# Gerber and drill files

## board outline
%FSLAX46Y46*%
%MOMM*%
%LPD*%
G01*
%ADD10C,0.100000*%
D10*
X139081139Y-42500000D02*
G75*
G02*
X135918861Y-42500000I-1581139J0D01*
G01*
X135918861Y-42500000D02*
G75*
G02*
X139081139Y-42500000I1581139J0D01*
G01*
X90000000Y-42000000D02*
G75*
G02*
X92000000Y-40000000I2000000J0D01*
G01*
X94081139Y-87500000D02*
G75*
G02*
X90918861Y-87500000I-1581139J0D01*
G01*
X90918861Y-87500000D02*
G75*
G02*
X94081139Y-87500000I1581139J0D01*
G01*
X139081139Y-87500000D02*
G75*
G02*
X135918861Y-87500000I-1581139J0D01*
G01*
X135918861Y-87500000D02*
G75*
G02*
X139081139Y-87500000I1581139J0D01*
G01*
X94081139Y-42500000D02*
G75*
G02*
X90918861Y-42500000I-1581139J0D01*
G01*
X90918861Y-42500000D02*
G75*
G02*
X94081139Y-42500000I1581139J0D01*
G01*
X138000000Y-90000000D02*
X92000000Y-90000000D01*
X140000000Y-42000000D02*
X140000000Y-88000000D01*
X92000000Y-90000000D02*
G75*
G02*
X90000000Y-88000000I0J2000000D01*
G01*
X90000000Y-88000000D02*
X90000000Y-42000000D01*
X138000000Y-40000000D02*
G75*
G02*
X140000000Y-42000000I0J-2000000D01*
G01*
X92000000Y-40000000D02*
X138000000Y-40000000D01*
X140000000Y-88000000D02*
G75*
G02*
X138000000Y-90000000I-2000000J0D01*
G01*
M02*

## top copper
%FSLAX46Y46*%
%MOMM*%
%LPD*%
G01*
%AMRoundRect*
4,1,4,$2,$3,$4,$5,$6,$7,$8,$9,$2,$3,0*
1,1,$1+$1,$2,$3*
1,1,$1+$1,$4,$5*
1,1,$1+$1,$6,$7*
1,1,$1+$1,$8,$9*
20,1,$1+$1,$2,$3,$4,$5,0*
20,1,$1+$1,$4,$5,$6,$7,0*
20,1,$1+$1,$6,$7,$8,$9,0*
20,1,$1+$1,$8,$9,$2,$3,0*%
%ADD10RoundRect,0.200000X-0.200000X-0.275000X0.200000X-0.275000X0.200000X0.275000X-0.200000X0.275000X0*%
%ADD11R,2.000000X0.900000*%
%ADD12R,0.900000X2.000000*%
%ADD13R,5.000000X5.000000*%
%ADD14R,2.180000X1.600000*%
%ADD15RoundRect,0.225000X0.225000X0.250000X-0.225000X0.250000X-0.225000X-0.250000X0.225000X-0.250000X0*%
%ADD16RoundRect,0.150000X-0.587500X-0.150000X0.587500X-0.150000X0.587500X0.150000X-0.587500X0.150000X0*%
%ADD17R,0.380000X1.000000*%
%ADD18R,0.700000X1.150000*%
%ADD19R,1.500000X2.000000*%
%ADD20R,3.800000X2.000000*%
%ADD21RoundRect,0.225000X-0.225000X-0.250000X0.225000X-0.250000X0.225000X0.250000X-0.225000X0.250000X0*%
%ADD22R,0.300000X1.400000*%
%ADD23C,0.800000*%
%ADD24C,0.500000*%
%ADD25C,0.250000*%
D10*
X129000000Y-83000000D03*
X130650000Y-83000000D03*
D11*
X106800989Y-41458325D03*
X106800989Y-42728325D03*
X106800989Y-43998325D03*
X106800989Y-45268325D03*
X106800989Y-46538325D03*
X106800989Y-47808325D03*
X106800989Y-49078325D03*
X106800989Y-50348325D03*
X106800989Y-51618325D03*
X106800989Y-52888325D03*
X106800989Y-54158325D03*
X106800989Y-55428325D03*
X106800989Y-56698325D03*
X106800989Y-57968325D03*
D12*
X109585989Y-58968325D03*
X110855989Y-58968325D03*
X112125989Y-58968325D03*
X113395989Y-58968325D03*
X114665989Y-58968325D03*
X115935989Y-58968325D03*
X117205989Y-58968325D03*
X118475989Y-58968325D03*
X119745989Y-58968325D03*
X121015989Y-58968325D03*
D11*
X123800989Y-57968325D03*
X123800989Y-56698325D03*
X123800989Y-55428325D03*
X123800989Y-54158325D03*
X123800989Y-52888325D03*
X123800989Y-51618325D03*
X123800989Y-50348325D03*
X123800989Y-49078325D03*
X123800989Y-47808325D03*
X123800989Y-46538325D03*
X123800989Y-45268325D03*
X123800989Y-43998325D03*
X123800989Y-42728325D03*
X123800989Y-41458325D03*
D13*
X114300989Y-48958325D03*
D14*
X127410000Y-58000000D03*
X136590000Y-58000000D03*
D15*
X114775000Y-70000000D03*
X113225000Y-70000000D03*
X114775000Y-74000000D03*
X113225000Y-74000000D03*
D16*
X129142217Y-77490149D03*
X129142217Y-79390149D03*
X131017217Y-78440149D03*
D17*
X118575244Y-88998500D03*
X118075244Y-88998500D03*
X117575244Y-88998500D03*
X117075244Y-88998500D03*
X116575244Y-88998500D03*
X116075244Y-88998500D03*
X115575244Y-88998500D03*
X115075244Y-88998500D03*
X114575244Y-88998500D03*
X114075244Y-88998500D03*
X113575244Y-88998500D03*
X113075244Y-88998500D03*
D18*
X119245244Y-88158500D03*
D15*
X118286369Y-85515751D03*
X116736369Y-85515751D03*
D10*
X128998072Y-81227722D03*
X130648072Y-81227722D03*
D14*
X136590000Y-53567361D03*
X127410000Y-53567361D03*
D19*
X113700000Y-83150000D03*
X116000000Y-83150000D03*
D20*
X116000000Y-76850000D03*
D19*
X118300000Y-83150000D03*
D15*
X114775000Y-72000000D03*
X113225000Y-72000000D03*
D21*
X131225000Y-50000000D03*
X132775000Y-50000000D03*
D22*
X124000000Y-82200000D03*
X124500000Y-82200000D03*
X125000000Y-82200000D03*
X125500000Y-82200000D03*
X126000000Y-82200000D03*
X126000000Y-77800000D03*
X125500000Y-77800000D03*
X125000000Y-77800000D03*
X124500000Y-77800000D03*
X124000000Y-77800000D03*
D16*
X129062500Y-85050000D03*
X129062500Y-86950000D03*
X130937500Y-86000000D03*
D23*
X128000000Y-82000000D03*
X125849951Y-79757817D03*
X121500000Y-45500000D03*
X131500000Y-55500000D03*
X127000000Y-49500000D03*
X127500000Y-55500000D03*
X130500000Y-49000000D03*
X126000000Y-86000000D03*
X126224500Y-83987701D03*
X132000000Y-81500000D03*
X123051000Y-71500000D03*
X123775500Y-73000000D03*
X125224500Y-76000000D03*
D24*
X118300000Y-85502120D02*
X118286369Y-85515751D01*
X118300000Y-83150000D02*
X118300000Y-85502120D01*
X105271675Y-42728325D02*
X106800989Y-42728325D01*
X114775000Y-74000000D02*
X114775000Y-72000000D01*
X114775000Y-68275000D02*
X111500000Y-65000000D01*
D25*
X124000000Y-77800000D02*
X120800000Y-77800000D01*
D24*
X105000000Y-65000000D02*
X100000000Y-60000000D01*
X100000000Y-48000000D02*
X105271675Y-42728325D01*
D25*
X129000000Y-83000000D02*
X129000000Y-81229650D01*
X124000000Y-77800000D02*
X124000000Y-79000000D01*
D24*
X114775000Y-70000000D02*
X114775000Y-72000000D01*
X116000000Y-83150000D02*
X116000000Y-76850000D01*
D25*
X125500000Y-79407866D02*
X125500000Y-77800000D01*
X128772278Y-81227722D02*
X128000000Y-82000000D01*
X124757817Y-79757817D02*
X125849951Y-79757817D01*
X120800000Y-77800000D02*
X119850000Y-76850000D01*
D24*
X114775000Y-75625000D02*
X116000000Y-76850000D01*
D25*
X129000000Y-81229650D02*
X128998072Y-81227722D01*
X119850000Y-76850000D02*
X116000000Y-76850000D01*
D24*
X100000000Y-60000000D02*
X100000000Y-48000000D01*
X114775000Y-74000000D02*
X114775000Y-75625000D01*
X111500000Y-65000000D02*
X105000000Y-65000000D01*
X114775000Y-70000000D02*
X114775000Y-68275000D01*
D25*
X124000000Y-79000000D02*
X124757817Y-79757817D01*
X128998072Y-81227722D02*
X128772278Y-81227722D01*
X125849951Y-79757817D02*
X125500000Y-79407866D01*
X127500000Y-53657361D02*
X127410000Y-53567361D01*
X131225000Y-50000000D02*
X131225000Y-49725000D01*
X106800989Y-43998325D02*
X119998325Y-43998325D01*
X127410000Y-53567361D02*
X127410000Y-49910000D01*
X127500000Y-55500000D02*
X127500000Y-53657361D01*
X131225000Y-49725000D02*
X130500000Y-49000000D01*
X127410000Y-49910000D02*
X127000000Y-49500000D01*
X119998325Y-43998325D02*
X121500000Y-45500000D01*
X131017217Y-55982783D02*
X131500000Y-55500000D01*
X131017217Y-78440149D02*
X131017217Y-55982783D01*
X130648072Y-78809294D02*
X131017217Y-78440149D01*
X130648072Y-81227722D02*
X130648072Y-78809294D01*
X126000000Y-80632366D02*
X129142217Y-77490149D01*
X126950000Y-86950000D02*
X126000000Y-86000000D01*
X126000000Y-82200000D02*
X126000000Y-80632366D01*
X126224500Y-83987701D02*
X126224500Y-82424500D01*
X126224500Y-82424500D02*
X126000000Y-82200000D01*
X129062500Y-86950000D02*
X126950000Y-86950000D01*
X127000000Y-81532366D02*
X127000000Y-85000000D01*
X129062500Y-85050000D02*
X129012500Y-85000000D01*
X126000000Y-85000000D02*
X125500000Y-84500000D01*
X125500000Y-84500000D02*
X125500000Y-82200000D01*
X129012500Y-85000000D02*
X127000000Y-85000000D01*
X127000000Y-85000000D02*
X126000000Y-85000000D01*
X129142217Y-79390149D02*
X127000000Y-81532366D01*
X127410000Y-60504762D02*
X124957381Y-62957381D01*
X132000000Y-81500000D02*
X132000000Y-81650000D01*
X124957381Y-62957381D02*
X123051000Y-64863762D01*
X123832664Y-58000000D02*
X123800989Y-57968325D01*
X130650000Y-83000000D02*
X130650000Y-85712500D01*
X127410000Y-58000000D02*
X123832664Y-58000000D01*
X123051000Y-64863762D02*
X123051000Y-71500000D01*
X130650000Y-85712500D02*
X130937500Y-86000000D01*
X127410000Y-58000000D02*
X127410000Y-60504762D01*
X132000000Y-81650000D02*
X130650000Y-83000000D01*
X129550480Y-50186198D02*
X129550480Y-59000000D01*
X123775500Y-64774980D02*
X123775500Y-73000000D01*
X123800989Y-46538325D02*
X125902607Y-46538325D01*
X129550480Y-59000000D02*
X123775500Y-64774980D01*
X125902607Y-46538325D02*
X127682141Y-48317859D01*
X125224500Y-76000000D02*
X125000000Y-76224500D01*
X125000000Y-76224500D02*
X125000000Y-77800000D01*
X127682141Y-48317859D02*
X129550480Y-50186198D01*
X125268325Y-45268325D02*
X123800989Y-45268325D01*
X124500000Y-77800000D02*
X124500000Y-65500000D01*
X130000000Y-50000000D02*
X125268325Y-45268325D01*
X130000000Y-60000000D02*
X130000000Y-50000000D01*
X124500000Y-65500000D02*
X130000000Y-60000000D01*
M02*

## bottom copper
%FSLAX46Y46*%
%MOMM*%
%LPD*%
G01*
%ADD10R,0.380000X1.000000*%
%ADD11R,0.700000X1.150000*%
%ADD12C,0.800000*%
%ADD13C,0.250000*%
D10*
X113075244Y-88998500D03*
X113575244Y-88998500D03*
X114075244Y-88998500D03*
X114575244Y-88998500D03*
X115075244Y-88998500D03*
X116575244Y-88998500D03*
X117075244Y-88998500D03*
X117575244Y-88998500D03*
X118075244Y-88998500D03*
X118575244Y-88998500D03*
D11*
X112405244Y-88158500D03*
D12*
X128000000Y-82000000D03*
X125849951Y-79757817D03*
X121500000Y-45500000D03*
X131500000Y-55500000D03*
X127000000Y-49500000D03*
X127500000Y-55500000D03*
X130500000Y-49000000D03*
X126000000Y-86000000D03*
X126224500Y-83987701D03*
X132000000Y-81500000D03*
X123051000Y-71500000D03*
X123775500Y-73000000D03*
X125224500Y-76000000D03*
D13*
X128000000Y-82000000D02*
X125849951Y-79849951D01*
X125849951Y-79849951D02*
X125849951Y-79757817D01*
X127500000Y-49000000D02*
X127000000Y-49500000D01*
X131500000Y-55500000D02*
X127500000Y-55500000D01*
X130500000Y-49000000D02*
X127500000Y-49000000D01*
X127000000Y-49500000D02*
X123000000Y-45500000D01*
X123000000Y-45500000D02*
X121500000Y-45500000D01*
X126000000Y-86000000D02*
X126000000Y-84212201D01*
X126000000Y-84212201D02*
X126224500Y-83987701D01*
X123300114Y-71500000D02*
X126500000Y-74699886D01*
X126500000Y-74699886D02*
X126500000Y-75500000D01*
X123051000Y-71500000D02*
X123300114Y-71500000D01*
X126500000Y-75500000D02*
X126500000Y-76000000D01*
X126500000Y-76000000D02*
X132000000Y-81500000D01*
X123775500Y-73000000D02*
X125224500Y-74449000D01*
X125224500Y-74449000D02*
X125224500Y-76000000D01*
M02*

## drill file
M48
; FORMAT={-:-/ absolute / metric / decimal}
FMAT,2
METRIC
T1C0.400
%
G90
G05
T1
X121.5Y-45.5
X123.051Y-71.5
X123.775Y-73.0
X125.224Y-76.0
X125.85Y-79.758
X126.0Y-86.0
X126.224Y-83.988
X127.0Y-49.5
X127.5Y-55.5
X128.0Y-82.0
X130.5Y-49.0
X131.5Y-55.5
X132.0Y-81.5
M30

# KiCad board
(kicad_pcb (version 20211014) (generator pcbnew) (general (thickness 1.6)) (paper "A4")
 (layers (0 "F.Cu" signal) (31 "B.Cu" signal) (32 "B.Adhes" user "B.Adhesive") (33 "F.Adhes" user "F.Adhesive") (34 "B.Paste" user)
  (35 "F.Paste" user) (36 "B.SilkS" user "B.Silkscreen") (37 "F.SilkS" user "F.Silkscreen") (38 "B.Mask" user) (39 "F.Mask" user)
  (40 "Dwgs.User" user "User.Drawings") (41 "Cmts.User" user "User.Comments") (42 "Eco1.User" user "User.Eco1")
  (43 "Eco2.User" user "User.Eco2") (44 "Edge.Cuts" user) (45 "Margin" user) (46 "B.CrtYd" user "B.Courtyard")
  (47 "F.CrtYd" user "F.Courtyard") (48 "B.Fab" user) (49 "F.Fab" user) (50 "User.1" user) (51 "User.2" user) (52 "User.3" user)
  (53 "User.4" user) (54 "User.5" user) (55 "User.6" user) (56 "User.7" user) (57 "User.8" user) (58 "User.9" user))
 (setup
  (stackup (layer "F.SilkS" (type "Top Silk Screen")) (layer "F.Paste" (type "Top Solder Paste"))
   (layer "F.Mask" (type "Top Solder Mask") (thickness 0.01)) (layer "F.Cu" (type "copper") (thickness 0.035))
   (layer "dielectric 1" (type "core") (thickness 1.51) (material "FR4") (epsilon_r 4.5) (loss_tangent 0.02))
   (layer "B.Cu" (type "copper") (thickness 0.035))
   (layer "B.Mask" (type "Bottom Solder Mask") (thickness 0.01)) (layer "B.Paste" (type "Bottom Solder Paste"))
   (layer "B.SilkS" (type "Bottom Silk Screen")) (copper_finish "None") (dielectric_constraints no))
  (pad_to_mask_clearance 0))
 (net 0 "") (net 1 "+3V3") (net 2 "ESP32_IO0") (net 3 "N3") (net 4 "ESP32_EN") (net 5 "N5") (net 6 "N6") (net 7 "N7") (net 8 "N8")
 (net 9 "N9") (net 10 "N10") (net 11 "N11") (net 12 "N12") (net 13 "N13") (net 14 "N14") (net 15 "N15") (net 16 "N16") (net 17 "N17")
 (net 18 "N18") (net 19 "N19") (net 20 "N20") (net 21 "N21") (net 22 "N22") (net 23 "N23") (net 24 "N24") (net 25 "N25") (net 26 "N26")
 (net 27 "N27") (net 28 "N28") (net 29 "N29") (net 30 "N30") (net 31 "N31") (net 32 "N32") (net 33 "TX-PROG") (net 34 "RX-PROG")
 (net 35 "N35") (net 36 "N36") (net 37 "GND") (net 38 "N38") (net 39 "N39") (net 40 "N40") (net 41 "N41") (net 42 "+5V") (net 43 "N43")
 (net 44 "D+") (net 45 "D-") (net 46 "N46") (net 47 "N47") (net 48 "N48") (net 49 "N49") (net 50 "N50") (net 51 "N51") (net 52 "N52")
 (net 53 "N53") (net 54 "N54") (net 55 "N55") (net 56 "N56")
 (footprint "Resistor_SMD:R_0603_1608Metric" (layer "F.Cu") (at 129.825 83)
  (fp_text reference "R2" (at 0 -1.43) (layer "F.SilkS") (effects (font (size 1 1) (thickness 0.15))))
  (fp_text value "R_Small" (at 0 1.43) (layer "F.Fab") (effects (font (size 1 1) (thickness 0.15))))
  (pad "1" smd roundrect (at -0.825 0) (size 0.8 0.95) (layers "F.Cu" "F.Paste" "F.Mask") (roundrect_rratio 0.25) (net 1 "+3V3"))
  (pad "2" smd roundrect (at 0.825 0) (size 0.8 0.95) (layers "F.Cu" "F.Paste" "F.Mask") (roundrect_rratio 0.25) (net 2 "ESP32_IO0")))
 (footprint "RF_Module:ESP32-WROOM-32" (layer "F.Cu") (at 115.300989 49.713325)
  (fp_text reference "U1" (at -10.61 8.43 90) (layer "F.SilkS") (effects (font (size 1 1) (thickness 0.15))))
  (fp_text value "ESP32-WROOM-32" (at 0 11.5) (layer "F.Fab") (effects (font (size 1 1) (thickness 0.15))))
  (pad "1" smd rect (at -8.5 -8.255) (size 2 0.9) (layers "F.Cu" "F.Paste" "F.Mask") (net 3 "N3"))
  (pad "2" smd rect (at -8.5 -6.985) (size 2 0.9) (layers "F.Cu" "F.Paste" "F.Mask") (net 1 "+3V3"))
  (pad "3" smd rect (at -8.5 -5.715) (size 2 0.9) (layers "F.Cu" "F.Paste" "F.Mask") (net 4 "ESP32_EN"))
  (pad "4" smd rect (at -8.5 -4.445) (size 2 0.9) (layers "F.Cu" "F.Paste" "F.Mask") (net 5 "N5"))
  (pad "5" smd rect (at -8.5 -3.175) (size 2 0.9) (layers "F.Cu" "F.Paste" "F.Mask") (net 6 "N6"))
  (pad "6" smd rect (at -8.5 -1.905) (size 2 0.9) (layers "F.Cu" "F.Paste" "F.Mask") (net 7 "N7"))
  (pad "7" smd rect (at -8.5 -0.635) (size 2 0.9) (layers "F.Cu" "F.Paste" "F.Mask") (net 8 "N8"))
  (pad "8" smd rect (at -8.5 0.635) (size 2 0.9) (layers "F.Cu" "F.Paste" "F.Mask") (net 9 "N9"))
  (pad "9" smd rect (at -8.5 1.905) (size 2 0.9) (layers "F.Cu" "F.Paste" "F.Mask") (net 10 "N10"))
  (pad "10" smd rect (at -8.5 3.175) (size 2 0.9) (layers "F.Cu" "F.Paste" "F.Mask") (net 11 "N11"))
  (pad "11" smd rect (at -8.5 4.445) (size 2 0.9) (layers "F.Cu" "F.Paste" "F.Mask") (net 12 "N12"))
  (pad "12" smd rect (at -8.5 5.715) (size 2 0.9) (layers "F.Cu" "F.Paste" "F.Mask") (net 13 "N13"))
  (pad "13" smd rect (at -8.5 6.985) (size 2 0.9) (layers "F.Cu" "F.Paste" "F.Mask") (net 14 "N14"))
  (pad "14" smd rect (at -8.5 8.255) (size 2 0.9) (layers "F.Cu" "F.Paste" "F.Mask") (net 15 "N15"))
  (pad "15" smd rect (at -5.715 9.255 90) (size 2 0.9) (layers "F.Cu" "F.Paste" "F.Mask") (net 3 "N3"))
  (pad "16" smd rect (at -4.445 9.255 90) (size 2 0.9) (layers "F.Cu" "F.Paste" "F.Mask") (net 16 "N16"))
  (pad "17" smd rect (at -3.175 9.255 90) (size 2 0.9) (layers "F.Cu" "F.Paste" "F.Mask") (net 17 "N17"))
  (pad "18" smd rect (at -1.905 9.255 90) (size 2 0.9) (layers "F.Cu" "F.Paste" "F.Mask") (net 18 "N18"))
  (pad "19" smd rect (at -0.635 9.255 90) (size 2 0.9) (layers "F.Cu" "F.Paste" "F.Mask") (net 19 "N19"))
  (pad "20" smd rect (at 0.635 9.255 90) (size 2 0.9) (layers "F.Cu" "F.Paste" "F.Mask") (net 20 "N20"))
  (pad "21" smd rect (at 1.905 9.255 90) (size 2 0.9) (layers "F.Cu" "F.Paste" "F.Mask") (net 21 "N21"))
  (pad "22" smd rect (at 3.175 9.255 90) (size 2 0.9) (layers "F.Cu" "F.Paste" "F.Mask") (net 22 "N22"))
  (pad "23" smd rect (at 4.445 9.255 90) (size 2 0.9) (layers "F.Cu" "F.Paste" "F.Mask") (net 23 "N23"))
  (pad "24" smd rect (at 5.715 9.255 90) (size 2 0.9) (layers "F.Cu" "F.Paste" "F.Mask") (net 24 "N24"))
  (pad "25" smd rect (at 8.5 8.255) (size 2 0.9) (layers "F.Cu" "F.Paste" "F.Mask") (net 2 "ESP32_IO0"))
  (pad "26" smd rect (at 8.5 6.985) (size 2 0.9) (layers "F.Cu" "F.Paste" "F.Mask") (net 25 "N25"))
  (pad "27" smd rect (at 8.5 5.715) (size 2 0.9) (layers "F.Cu" "F.Paste" "F.Mask") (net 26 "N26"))
  (pad "28" smd rect (at 8.5 4.445) (size 2 0.9) (layers "F.Cu" "F.Paste" "F.Mask") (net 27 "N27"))
  (pad "29" smd rect (at 8.5 3.175) (size 2 0.9) (layers "F.Cu" "F.Paste" "F.Mask") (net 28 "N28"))
  (pad "30" smd rect (at 8.5 1.905) (size 2 0.9) (layers "F.Cu" "F.Paste" "F.Mask") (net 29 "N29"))
  (pad "31" smd rect (at 8.5 0.635) (size 2 0.9) (layers "F.Cu" "F.Paste" "F.Mask") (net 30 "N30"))
  (pad "32" smd rect (at 8.5 -0.635) (size 2 0.9) (layers "F.Cu" "F.Paste" "F.Mask") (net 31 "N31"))
  (pad "33" smd rect (at 8.5 -1.905) (size 2 0.9) (layers "F.Cu" "F.Paste" "F.Mask") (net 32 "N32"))
  (pad "34" smd rect (at 8.5 -3.175) (size 2 0.9) (layers "F.Cu" "F.Paste" "F.Mask") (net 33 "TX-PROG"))
  (pad "35" smd rect (at 8.5 -4.445) (size 2 0.9) (layers "F.Cu" "F.Paste" "F.Mask") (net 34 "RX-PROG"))
  (pad "36" smd rect (at 8.5 -5.715) (size 2 0.9) (layers "F.Cu" "F.Paste" "F.Mask") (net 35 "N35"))
  (pad "37" smd rect (at 8.5 -6.985) (size 2 0.9) (layers "F.Cu" "F.Paste" "F.Mask") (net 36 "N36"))
  (pad "38" smd rect (at 8.5 -8.255) (size 2 0.9) (layers "F.Cu" "F.Paste" "F.Mask") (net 3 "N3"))
  (pad "39" smd rect (at -1 -0.755) (size 5 5) (layers "F.Cu" "F.Paste" "F.Mask") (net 3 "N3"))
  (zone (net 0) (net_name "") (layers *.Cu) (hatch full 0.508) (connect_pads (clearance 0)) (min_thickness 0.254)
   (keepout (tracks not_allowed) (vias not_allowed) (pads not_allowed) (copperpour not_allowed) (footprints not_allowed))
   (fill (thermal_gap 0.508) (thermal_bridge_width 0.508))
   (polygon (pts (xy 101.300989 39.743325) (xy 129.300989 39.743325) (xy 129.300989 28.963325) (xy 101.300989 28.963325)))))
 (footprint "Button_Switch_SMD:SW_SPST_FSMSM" (layer "F.Cu") (at 132 58)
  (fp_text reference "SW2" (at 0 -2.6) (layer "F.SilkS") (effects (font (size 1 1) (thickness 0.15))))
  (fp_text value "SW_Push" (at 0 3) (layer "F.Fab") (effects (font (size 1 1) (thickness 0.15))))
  (pad "1" smd rect (at -4.59 0) (size 2.18 1.6) (layers "F.Cu" "F.Paste" "F.Mask") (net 2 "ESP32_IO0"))
  (pad "2" smd rect (at 4.59 0) (size 2.18 1.6) (layers "F.Cu" "F.Paste" "F.Mask") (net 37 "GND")))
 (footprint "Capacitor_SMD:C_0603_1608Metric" (layer "F.Cu") (at 114 70 180)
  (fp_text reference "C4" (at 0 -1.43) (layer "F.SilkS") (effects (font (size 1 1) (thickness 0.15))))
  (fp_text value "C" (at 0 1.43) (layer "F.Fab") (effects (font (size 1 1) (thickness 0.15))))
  (pad "1" smd roundrect (at -0.775 0 180) (size 0.9 0.95) (layers "F.Cu" "F.Paste" "F.Mask") (roundrect_rratio 0.25) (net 1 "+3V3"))
  (pad "2" smd roundrect (at 0.775 0 180) (size 0.9 0.95) (layers "F.Cu" "F.Paste" "F.Mask") (roundrect_rratio 0.25) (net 37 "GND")))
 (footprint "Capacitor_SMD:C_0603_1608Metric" (layer "F.Cu") (at 114 74 180)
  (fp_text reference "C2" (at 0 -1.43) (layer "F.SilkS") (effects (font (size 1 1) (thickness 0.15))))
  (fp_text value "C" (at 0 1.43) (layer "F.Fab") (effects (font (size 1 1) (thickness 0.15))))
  (pad "1" smd roundrect (at -0.775 0 180) (size 0.9 0.95) (layers "F.Cu" "F.Paste" "F.Mask") (roundrect_rratio 0.25) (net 1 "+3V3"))
  (pad "2" smd roundrect (at 0.775 0 180) (size 0.9 0.95) (layers "F.Cu" "F.Paste" "F.Mask") (roundrect_rratio 0.25) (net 37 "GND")))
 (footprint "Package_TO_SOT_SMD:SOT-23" (layer "F.Cu") (at 130.079717 78.440149)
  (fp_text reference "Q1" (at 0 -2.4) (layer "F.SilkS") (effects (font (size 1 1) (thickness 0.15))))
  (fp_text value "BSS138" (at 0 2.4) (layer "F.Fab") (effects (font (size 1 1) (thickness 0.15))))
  (pad "1" smd roundrect (at -0.9375 -0.95) (size 1.475 0.6) (layers "F.Cu" "F.Paste" "F.Mask") (roundrect_rratio 0.25) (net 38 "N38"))
  (pad "2" smd roundrect (at -0.9375 0.95) (size 1.475 0.6) (layers "F.Cu" "F.Paste" "F.Mask") (roundrect_rratio 0.25) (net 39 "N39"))
  (pad "3" smd roundrect (at 0.9375 0) (size 1.475 0.6) (layers "F.Cu" "F.Paste" "F.Mask") (roundrect_rratio 0.25) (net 4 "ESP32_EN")))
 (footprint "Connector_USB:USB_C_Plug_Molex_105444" (layer "F.Cu") (at 115.825244 89.0385 180)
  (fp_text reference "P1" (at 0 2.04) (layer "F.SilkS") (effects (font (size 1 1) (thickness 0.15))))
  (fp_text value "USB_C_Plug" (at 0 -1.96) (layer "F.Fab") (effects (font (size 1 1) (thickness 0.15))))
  (pad "A1" smd rect (at -2.75 0.04 180) (size 0.38 1) (layers "F.Cu" "F.Paste" "F.Mask") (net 37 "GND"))
  (pad "A2" smd rect (at -2.25 0.04 180) (size 0.38 1) (layers "F.Cu" "F.Paste" "F.Mask") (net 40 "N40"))
  (pad "A3" smd rect (at -1.75 0.04 180) (size 0.38 1) (layers "F.Cu" "F.Paste" "F.Mask") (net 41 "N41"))
  (pad "A4" smd rect (at -1.25 0.04 180) (size 0.38 1) (layers "F.Cu" "F.Paste" "F.Mask") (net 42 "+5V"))
  (pad "A5" smd rect (at -0.75 0.04 180) (size 0.38 1) (layers "F.Cu" "F.Paste" "F.Mask") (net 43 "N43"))
  (pad "A6" smd rect (at -0.25 0.04 180) (size 0.38 1) (layers "F.Cu" "F.Paste" "F.Mask") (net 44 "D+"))
  (pad "A7" smd rect (at 0.25 0.04 180) (size 0.38 1) (layers "F.Cu" "F.Paste" "F.Mask") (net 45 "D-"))
  (pad "A8" smd rect (at 0.75 0.04 180) (size 0.38 1) (layers "F.Cu" "F.Paste" "F.Mask") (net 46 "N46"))
  (pad "A9" smd rect (at 1.25 0.04 180) (size 0.38 1) (layers "F.Cu" "F.Paste" "F.Mask") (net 42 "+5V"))
  (pad "A10" smd rect (at 1.75 0.04 180) (size 0.38 1) (layers "F.Cu" "F.Paste" "F.Mask") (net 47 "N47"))
  (pad "A11" smd rect (at 2.25 0.04 180) (size 0.38 1) (layers "F.Cu" "F.Paste" "F.Mask") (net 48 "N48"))
  (pad "A12" smd rect (at 2.75 0.04 180) (size 0.38 1) (layers "F.Cu" "F.Paste" "F.Mask") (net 37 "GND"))
  (pad "B1" smd rect (at 2.75 0.04 180) (size 0.38 1) (layers "B.Cu" "B.Paste" "B.Mask") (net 37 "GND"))
  (pad "B2" smd rect (at 2.25 0.04 180) (size 0.38 1) (layers "B.Cu" "B.Paste" "B.Mask") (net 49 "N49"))
  (pad "B3" smd rect (at 1.75 0.04 180) (size 0.38 1) (layers "B.Cu" "B.Paste" "B.Mask") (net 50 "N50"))
  (pad "B4" smd rect (at 1.25 0.04 180) (size 0.38 1) (layers "B.Cu" "B.Paste" "B.Mask") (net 42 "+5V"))
  (pad "B5" smd rect (at 0.75 0.04 180) (size 0.38 1) (layers "B.Cu" "B.Paste" "B.Mask") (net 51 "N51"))
  (pad "B8" smd rect (at -0.75 0.04 180) (size 0.38 1) (layers "B.Cu" "B.Paste" "B.Mask") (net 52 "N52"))
  (pad "B9" smd rect (at -1.25 0.04 180) (size 0.38 1) (layers "B.Cu" "B.Paste" "B.Mask") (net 42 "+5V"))
  (pad "B10" smd rect (at -1.75 0.04 180) (size 0.38 1) (layers "B.Cu" "B.Paste" "B.Mask") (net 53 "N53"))
  (pad "B11" smd rect (at -2.25 0.04 180) (size 0.38 1) (layers "B.Cu" "B.Paste" "B.Mask") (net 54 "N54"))
  (pad "B12" smd rect (at -2.75 0.04 180) (size 0.38 1) (layers "B.Cu" "B.Paste" "B.Mask") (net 37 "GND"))
  (pad "S1" smd rect (at 3.42 0.88 180) (size 0.7 1.15) (layers "B.Cu" "B.Paste" "B.Mask") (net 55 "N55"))
  (pad "S1" smd rect (at -3.42 0.88 180) (size 0.7 1.15) (layers "F.Cu" "F.Paste" "F.Mask") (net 55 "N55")))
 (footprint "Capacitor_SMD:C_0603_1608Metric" (layer "F.Cu") (at 117.511369 85.515751 180)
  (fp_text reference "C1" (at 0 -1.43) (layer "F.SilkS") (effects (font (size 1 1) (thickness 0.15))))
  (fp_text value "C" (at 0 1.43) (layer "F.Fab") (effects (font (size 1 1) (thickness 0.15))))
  (pad "1" smd roundrect (at -0.775 0 180) (size 0.9 0.95) (layers "F.Cu" "F.Paste" "F.Mask") (roundrect_rratio 0.25) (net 42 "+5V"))
  (pad "2" smd roundrect (at 0.775 0 180) (size 0.9 0.95) (layers "F.Cu" "F.Paste" "F.Mask") (roundrect_rratio 0.25) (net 37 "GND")))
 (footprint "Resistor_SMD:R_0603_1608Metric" (layer "F.Cu") (at 129.823072 81.227722)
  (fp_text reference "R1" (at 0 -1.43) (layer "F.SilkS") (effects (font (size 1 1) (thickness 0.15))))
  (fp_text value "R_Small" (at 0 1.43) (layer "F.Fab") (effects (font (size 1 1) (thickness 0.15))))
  (pad "1" smd roundrect (at -0.825 0) (size 0.8 0.95) (layers "F.Cu" "F.Paste" "F.Mask") (roundrect_rratio 0.25) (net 1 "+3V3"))
  (pad "2" smd roundrect (at 0.825 0) (size 0.8 0.95) (layers "F.Cu" "F.Paste" "F.Mask") (roundrect_rratio 0.25) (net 4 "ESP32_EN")))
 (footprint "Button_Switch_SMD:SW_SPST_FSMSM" (layer "F.Cu") (at 132 53.567361 180)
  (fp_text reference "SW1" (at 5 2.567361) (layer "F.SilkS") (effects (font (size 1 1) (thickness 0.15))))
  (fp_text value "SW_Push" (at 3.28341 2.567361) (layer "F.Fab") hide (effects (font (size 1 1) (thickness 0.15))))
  (pad "1" smd rect (at -4.59 0 180) (size 2.18 1.6) (layers "F.Cu" "F.Paste" "F.Mask") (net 37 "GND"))
  (pad "2" smd rect (at 4.59 0 180) (size 2.18 1.6) (layers "F.Cu" "F.Paste" "F.Mask") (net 4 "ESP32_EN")))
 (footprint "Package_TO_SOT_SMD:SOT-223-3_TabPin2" (layer "F.Cu") (at 116 80 90)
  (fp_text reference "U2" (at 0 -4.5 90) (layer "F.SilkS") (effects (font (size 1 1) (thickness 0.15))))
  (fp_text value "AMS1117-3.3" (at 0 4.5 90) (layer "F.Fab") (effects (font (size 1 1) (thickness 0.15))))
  (pad "1" smd rect (at -3.15 -2.3 90) (size 2 1.5) (layers "F.Cu" "F.Paste" "F.Mask") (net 37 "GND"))
  (pad "2" smd rect (at -3.15 0 90) (size 2 1.5) (layers "F.Cu" "F.Paste" "F.Mask") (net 1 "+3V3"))
  (pad "2" smd rect (at 3.15 0 90) (size 2 3.8) (layers "F.Cu" "F.Paste" "F.Mask") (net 1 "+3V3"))
  (pad "3" smd rect (at -3.15 2.3 90) (size 2 1.5) (layers "F.Cu" "F.Paste" "F.Mask") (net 42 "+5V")))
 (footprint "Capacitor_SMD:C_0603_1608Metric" (layer "F.Cu") (at 114 72 180)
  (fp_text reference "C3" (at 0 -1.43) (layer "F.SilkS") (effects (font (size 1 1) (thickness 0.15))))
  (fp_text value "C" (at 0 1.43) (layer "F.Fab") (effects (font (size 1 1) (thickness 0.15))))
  (pad "1" smd roundrect (at -0.775 0 180) (size 0.9 0.95) (layers "F.Cu" "F.Paste" "F.Mask") (roundrect_rratio 0.25) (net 1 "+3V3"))
  (pad "2" smd roundrect (at 0.775 0 180) (size 0.9 0.95) (layers "F.Cu" "F.Paste" "F.Mask") (roundrect_rratio 0.25) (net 37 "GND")))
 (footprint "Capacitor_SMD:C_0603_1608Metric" (layer "F.Cu") (at 132 50)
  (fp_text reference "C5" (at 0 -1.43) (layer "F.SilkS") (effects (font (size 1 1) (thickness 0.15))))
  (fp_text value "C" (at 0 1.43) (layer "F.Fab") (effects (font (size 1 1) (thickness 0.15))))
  (pad "1" smd roundrect (at -0.775 0) (size 0.9 0.95) (layers "F.Cu" "F.Paste" "F.Mask") (roundrect_rratio 0.25) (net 4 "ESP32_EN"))
  (pad "2" smd roundrect (at 0.775 0) (size 0.9 0.95) (layers "F.Cu" "F.Paste" "F.Mask") (roundrect_rratio 0.25) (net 37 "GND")))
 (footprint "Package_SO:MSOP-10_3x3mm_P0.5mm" (layer "F.Cu") (at 125 80 90)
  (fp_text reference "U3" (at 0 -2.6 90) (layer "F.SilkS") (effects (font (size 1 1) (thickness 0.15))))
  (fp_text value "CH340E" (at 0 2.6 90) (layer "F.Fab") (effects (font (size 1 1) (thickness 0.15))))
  (pad "1" smd rect (at -2.2 -1 90) (size 1.4 0.3) (layers "F.Cu" "F.Paste" "F.Mask") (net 45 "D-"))
  (pad "2" smd rect (at -2.2 -0.5 90) (size 1.4 0.3) (layers "F.Cu" "F.Paste" "F.Mask") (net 44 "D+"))
  (pad "3" smd rect (at -2.2 0 90) (size 1.4 0.3) (layers "F.Cu" "F.Paste" "F.Mask") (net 37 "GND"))
  (pad "4" smd rect (at -2.2 0.5 90) (size 1.4 0.3) (layers "F.Cu" "F.Paste" "F.Mask") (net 39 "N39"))
  (pad "5" smd rect (at -2.2 1 90) (size 1.4 0.3) (layers "F.Cu" "F.Paste" "F.Mask") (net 38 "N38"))
  (pad "6" smd rect (at 2.2 1 90) (size 1.4 0.3) (layers "F.Cu" "F.Paste" "F.Mask") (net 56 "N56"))
  (pad "7" smd rect (at 2.2 0.5 90) (size 1.4 0.3) (layers "F.Cu" "F.Paste" "F.Mask") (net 1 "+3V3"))
  (pad "8" smd rect (at 2.2 0 90) (size 1.4 0.3) (layers "F.Cu" "F.Paste" "F.Mask") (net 33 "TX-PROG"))
  (pad "9" smd rect (at 2.2 -0.5 90) (size 1.4 0.3) (layers "F.Cu" "F.Paste" "F.Mask") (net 34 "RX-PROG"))
  (pad "10" smd rect (at 2.2 -1 90) (size 1.4 0.3) (layers "F.Cu" "F.Paste" "F.Mask") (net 1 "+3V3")))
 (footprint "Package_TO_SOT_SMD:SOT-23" (layer "F.Cu") (at 130 86)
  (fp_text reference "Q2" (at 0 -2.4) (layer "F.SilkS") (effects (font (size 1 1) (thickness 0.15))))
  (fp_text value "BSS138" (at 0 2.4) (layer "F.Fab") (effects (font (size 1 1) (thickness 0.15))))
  (pad "1" smd roundrect (at -0.9375 -0.95) (size 1.475 0.6) (layers "F.Cu" "F.Paste" "F.Mask") (roundrect_rratio 0.25) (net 39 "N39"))
  (pad "2" smd roundrect (at -0.9375 0.95) (size 1.475 0.6) (layers "F.Cu" "F.Paste" "F.Mask") (roundrect_rratio 0.25) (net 38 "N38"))
  (pad "3" smd roundrect (at 0.9375 0) (size 1.475 0.6) (layers "F.Cu" "F.Paste" "F.Mask") (roundrect_rratio 0.25) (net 2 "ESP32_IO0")))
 (gr_circle (center 137.5 42.5) (end 139 43) (layer "Edge.Cuts") (width 0.1) (fill none))
 (gr_arc (start 90 42) (mid 90.585786 40.585786) (end 92 40) (layer "Edge.Cuts") (width 0.1))
 (gr_circle (center 92.5 87.5) (end 94 88) (layer "Edge.Cuts") (width 0.1) (fill none))
 (gr_circle (center 137.5 87.5) (end 139 88) (layer "Edge.Cuts") (width 0.1) (fill none))
 (gr_circle (center 92.5 42.5) (end 94 43) (layer "Edge.Cuts") (width 0.1) (fill none))
 (gr_line (start 138 90) (end 92 90) (layer "Edge.Cuts") (width 0.1))
 (gr_line (start 140 42) (end 140 88) (layer "Edge.Cuts") (width 0.1))
 (gr_arc (start 92 90) (mid 90.585786 89.414214) (end 90 88) (layer "Edge.Cuts") (width 0.1))
 (gr_line (start 90 88) (end 90 42) (layer "Edge.Cuts") (width 0.1))
 (gr_arc (start 138 40) (mid 139.414214 40.585786) (end 140 42) (layer "Edge.Cuts") (width 0.1))
 (gr_line (start 92 40) (end 138 40) (layer "Edge.Cuts") (width 0.1))
 (gr_arc (start 140 88) (mid 139.414214 89.414214) (end 138 90) (layer "Edge.Cuts") (width 0.1))
 (segment (start 118.3 85.50212) (end 118.286369 85.515751) (width 0.5) (layer "F.Cu") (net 42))
 (segment (start 118.3 83.15) (end 118.3 85.50212) (width 0.5) (layer "F.Cu") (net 42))
 (segment (start 105.271675 42.728325) (end 106.800989 42.728325) (width 0.5) (layer "F.Cu") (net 1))
 (segment (start 114.775 74) (end 114.775 72) (width 0.5) (layer "F.Cu") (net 1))
 (segment (start 114.775 68.275) (end 111.5 65) (width 0.5) (layer "F.Cu") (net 1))
 (segment (start 124 77.8) (end 120.8 77.8) (width 0.25) (layer "F.Cu") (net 1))
 (segment (start 105 65) (end 100 60) (width 0.5) (layer "F.Cu") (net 1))
 (segment (start 100 48) (end 105.271675 42.728325) (width 0.5) (layer "F.Cu") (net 1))
 (segment (start 129 83) (end 129 81.22965) (width 0.25) (layer "F.Cu") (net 1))
 (segment (start 124 77.8) (end 124 79) (width 0.25) (layer "F.Cu") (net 1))
 (segment (start 114.775 70) (end 114.775 72) (width 0.5) (layer "F.Cu") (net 1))
 (segment (start 116 83.15) (end 116 76.85) (width 0.5) (layer "F.Cu") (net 1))
 (segment (start 125.5 79.407866) (end 125.5 77.8) (width 0.25) (layer "F.Cu") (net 1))
 (segment (start 128.772278 81.227722) (end 128 82) (width 0.25) (layer "F.Cu") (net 1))
 (segment (start 124.757817 79.757817) (end 125.849951 79.757817) (width 0.25) (layer "F.Cu") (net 1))
 (segment (start 120.8 77.8) (end 119.85 76.85) (width 0.25) (layer "F.Cu") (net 1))
 (segment (start 114.775 75.625) (end 116 76.85) (width 0.5) (layer "F.Cu") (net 1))
 (segment (start 129 81.22965) (end 128.998072 81.227722) (width 0.25) (layer "F.Cu") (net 1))
 (segment (start 119.85 76.85) (end 116 76.85) (width 0.25) (layer "F.Cu") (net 1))
 (segment (start 100 60) (end 100 48) (width 0.5) (layer "F.Cu") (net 1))
 (segment (start 114.775 74) (end 114.775 75.625) (width 0.5) (layer "F.Cu") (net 1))
 (segment (start 111.5 65) (end 105 65) (width 0.5) (layer "F.Cu") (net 1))
 (segment (start 114.775 70) (end 114.775 68.275) (width 0.5) (layer "F.Cu") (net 1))
 (segment (start 124 79) (end 124.757817 79.757817) (width 0.25) (layer "F.Cu") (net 1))
 (segment (start 128.998072 81.227722) (end 128.772278 81.227722) (width 0.25) (layer "F.Cu") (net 1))
 (segment (start 125.849951 79.757817) (end 125.5 79.407866) (width 0.25) (layer "F.Cu") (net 1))
 (via (at 128 82) (size 0.8) (drill 0.4) (layers "F.Cu" "B.Cu") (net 1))
 (via (at 125.849951 79.757817) (size 0.8) (drill 0.4) (layers "F.Cu" "B.Cu") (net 1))
 (segment (start 128 82) (end 125.849951 79.849951) (width 0.25) (layer "B.Cu") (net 1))
 (segment (start 125.849951 79.849951) (end 125.849951 79.757817) (width 0.25) (layer "B.Cu") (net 1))
 (segment (start 127.5 53.657361) (end 127.41 53.567361) (width 0.25) (layer "F.Cu") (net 4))
 (segment (start 131.225 50) (end 131.225 49.725) (width 0.25) (layer "F.Cu") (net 4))
 (segment (start 106.800989 43.998325) (end 119.998325 43.998325) (width 0.25) (layer "F.Cu") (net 4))
 (segment (start 127.41 53.567361) (end 127.41 49.91) (width 0.25) (layer "F.Cu") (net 4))
 (segment (start 127.5 55.5) (end 127.5 53.657361) (width 0.25) (layer "F.Cu") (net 4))
 (segment (start 131.225 49.725) (end 130.5 49) (width 0.25) (layer "F.Cu") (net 4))
 (segment (start 127.41 49.91) (end 127 49.5) (width 0.25) (layer "F.Cu") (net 4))
 (segment (start 119.998325 43.998325) (end 121.5 45.5) (width 0.25) (layer "F.Cu") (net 4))
 (segment (start 131.017217 55.982783) (end 131.5 55.5) (width 0.25) (layer "F.Cu") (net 4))
 (segment (start 131.017217 78.440149) (end 131.017217 55.982783) (width 0.25) (layer "F.Cu") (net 4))
 (segment (start 130.648072 78.809294) (end 131.017217 78.440149) (width 0.25) (layer "F.Cu") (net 4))
 (segment (start 130.648072 81.227722) (end 130.648072 78.809294) (width 0.25) (layer "F.Cu") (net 4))
 (via (at 121.5 45.5) (size 0.8) (drill 0.4) (layers "F.Cu" "B.Cu") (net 4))
 (via (at 131.5 55.5) (size 0.8) (drill 0.4) (layers "F.Cu" "B.Cu") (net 4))
 (via (at 127 49.5) (size 0.8) (drill 0.4) (layers "F.Cu" "B.Cu") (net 4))
 (via (at 127.5 55.5) (size 0.8) (drill 0.4) (layers "F.Cu" "B.Cu") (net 4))
 (via (at 130.5 49) (size 0.8) (drill 0.4) (layers "F.Cu" "B.Cu") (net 4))
 (segment (start 127.5 49) (end 127 49.5) (width 0.25) (layer "B.Cu") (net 4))
 (segment (start 131.5 55.5) (end 127.5 55.5) (width 0.25) (layer "B.Cu") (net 4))
 (segment (start 130.5 49) (end 127.5 49) (width 0.25) (layer "B.Cu") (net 4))
 (segment (start 127 49.5) (end 123 45.5) (width 0.25) (layer "B.Cu") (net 4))
 (segment (start 123 45.5) (end 121.5 45.5) (width 0.25) (layer "B.Cu") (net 4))
 (segment (start 126 80.632366) (end 129.142217 77.490149) (width 0.25) (layer "F.Cu") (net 38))
 (segment (start 126.95 86.95) (end 126 86) (width 0.25) (layer "F.Cu") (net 38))
 (segment (start 126 82.2) (end 126 80.632366) (width 0.25) (layer "F.Cu") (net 38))
 (segment (start 126.2245 83.987701) (end 126.2245 82.4245) (width 0.25) (layer "F.Cu") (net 38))
 (segment (start 126.2245 82.4245) (end 126 82.2) (width 0.25) (layer "F.Cu") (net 38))
 (segment (start 129.0625 86.95) (end 126.95 86.95) (width 0.25) (layer "F.Cu") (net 38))
 (via (at 126 86) (size 0.8) (drill 0.4) (layers "F.Cu" "B.Cu") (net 38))
 (via (at 126.2245 83.987701) (size 0.8) (drill 0.4) (layers "F.Cu" "B.Cu") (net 38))
 (segment (start 126 86) (end 126 84.212201) (width 0.25) (layer "B.Cu") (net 38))
 (segment (start 126 84.212201) (end 126.2245 83.987701) (width 0.25) (layer "B.Cu") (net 38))
 (segment (start 127 81.532366) (end 127 85) (width 0.25) (layer "F.Cu") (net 39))
 (segment (start 129.0625 85.05) (end 129.0125 85) (width 0.25) (layer "F.Cu") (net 39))
 (segment (start 126 85) (end 125.5 84.5) (width 0.25) (layer "F.Cu") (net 39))
 (segment (start 125.5 84.5) (end 125.5 82.2) (width 0.25) (layer "F.Cu") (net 39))
 (segment (start 129.0125 85) (end 127 85) (width 0.25) (layer "F.Cu") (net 39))
 (segment (start 127 85) (end 126 85) (width 0.25) (layer "F.Cu") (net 39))
 (segment (start 129.142217 79.390149) (end 127 81.532366) (width 0.25) (layer "F.Cu") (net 39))
 (segment (start 127.41 60.504762) (end 124.957381 62.957381) (width 0.25) (layer "F.Cu") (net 2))
 (segment (start 132 81.5) (end 132 81.65) (width 0.25) (layer "F.Cu") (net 2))
 (segment (start 124.957381 62.957381) (end 123.051 64.863762) (width 0.25) (layer "F.Cu") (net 2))
 (segment (start 123.832664 58) (end 123.800989 57.968325) (width 0.25) (layer "F.Cu") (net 2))
 (segment (start 130.65 83) (end 130.65 85.7125) (width 0.25) (layer "F.Cu") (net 2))
 (segment (start 127.41 58) (end 123.832664 58) (width 0.25) (layer "F.Cu") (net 2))
 (segment (start 123.051 64.863762) (end 123.051 71.5) (width 0.25) (layer "F.Cu") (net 2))
 (segment (start 130.65 85.7125) (end 130.9375 86) (width 0.25) (layer "F.Cu") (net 2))
 (segment (start 127.41 58) (end 127.41 60.504762) (width 0.25) (layer "F.Cu") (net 2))
 (segment (start 132 81.65) (end 130.65 83) (width 0.25) (layer "F.Cu") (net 2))
 (via (at 132 81.5) (size 0.8) (drill 0.4) (layers "F.Cu" "B.Cu") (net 2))
 (via (at 123.051 71.5) (size 0.8) (drill 0.4) (layers "F.Cu" "B.Cu") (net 2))
 (segment (start 123.300114 71.5) (end 126.5 74.699886) (width 0.25) (layer "B.Cu") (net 2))
 (segment (start 126.5 74.699886) (end 126.5 75.5) (width 0.25) (layer "B.Cu") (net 2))
 (segment (start 123.051 71.5) (end 123.300114 71.5) (width 0.25) (layer "B.Cu") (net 2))
 (segment (start 126.5 75.5) (end 126.5 76) (width 0.25) (layer "B.Cu") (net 2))
 (segment (start 126.5 76) (end 132 81.5) (width 0.25) (layer "B.Cu") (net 2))
 (segment (start 129.55048 50.186198) (end 129.55048 59) (width 0.25) (layer "F.Cu") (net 33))
 (segment (start 123.7755 64.77498) (end 123.7755 73) (width 0.25) (layer "F.Cu") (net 33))
 (segment (start 123.800989 46.538325) (end 125.902607 46.538325) (width 0.25) (layer "F.Cu") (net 33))
 (segment (start 129.55048 59) (end 123.7755 64.77498) (width 0.25) (layer "F.Cu") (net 33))
 (segment (start 125.902607 46.538325) (end 127.682141 48.317859) (width 0.25) (layer "F.Cu") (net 33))
 (segment (start 125.2245 76) (end 125 76.2245) (width 0.25) (layer "F.Cu") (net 33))
 (segment (start 125 76.2245) (end 125 77.8) (width 0.25) (layer "F.Cu") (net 33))
 (segment (start 127.682141 48.317859) (end 129.55048 50.186198) (width 0.25) (layer "F.Cu") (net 33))
 (via (at 123.7755 73) (size 0.8) (drill 0.4) (layers "F.Cu" "B.Cu") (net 33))
 (via (at 125.2245 76) (size 0.8) (drill 0.4) (layers "F.Cu" "B.Cu") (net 33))
 (segment (start 123.7755 73) (end 125.2245 74.449) (width 0.25) (layer "B.Cu") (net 33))
 (segment (start 125.2245 74.449) (end 125.2245 76) (width 0.25) (layer "B.Cu") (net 33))
 (segment (start 125.268325 45.268325) (end 123.800989 45.268325) (width 0.25) (layer "F.Cu") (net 34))
 (segment (start 124.5 77.8) (end 124.5 65.5) (width 0.25) (layer "F.Cu") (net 34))
 (segment (start 130 50) (end 125.268325 45.268325) (width 0.25) (layer "F.Cu") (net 34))
 (segment (start 130 60) (end 130 50) (width 0.25) (layer "F.Cu") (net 34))
 (segment (start 124.5 65.5) (end 130 60) (width 0.25) (layer "F.Cu") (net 34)))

